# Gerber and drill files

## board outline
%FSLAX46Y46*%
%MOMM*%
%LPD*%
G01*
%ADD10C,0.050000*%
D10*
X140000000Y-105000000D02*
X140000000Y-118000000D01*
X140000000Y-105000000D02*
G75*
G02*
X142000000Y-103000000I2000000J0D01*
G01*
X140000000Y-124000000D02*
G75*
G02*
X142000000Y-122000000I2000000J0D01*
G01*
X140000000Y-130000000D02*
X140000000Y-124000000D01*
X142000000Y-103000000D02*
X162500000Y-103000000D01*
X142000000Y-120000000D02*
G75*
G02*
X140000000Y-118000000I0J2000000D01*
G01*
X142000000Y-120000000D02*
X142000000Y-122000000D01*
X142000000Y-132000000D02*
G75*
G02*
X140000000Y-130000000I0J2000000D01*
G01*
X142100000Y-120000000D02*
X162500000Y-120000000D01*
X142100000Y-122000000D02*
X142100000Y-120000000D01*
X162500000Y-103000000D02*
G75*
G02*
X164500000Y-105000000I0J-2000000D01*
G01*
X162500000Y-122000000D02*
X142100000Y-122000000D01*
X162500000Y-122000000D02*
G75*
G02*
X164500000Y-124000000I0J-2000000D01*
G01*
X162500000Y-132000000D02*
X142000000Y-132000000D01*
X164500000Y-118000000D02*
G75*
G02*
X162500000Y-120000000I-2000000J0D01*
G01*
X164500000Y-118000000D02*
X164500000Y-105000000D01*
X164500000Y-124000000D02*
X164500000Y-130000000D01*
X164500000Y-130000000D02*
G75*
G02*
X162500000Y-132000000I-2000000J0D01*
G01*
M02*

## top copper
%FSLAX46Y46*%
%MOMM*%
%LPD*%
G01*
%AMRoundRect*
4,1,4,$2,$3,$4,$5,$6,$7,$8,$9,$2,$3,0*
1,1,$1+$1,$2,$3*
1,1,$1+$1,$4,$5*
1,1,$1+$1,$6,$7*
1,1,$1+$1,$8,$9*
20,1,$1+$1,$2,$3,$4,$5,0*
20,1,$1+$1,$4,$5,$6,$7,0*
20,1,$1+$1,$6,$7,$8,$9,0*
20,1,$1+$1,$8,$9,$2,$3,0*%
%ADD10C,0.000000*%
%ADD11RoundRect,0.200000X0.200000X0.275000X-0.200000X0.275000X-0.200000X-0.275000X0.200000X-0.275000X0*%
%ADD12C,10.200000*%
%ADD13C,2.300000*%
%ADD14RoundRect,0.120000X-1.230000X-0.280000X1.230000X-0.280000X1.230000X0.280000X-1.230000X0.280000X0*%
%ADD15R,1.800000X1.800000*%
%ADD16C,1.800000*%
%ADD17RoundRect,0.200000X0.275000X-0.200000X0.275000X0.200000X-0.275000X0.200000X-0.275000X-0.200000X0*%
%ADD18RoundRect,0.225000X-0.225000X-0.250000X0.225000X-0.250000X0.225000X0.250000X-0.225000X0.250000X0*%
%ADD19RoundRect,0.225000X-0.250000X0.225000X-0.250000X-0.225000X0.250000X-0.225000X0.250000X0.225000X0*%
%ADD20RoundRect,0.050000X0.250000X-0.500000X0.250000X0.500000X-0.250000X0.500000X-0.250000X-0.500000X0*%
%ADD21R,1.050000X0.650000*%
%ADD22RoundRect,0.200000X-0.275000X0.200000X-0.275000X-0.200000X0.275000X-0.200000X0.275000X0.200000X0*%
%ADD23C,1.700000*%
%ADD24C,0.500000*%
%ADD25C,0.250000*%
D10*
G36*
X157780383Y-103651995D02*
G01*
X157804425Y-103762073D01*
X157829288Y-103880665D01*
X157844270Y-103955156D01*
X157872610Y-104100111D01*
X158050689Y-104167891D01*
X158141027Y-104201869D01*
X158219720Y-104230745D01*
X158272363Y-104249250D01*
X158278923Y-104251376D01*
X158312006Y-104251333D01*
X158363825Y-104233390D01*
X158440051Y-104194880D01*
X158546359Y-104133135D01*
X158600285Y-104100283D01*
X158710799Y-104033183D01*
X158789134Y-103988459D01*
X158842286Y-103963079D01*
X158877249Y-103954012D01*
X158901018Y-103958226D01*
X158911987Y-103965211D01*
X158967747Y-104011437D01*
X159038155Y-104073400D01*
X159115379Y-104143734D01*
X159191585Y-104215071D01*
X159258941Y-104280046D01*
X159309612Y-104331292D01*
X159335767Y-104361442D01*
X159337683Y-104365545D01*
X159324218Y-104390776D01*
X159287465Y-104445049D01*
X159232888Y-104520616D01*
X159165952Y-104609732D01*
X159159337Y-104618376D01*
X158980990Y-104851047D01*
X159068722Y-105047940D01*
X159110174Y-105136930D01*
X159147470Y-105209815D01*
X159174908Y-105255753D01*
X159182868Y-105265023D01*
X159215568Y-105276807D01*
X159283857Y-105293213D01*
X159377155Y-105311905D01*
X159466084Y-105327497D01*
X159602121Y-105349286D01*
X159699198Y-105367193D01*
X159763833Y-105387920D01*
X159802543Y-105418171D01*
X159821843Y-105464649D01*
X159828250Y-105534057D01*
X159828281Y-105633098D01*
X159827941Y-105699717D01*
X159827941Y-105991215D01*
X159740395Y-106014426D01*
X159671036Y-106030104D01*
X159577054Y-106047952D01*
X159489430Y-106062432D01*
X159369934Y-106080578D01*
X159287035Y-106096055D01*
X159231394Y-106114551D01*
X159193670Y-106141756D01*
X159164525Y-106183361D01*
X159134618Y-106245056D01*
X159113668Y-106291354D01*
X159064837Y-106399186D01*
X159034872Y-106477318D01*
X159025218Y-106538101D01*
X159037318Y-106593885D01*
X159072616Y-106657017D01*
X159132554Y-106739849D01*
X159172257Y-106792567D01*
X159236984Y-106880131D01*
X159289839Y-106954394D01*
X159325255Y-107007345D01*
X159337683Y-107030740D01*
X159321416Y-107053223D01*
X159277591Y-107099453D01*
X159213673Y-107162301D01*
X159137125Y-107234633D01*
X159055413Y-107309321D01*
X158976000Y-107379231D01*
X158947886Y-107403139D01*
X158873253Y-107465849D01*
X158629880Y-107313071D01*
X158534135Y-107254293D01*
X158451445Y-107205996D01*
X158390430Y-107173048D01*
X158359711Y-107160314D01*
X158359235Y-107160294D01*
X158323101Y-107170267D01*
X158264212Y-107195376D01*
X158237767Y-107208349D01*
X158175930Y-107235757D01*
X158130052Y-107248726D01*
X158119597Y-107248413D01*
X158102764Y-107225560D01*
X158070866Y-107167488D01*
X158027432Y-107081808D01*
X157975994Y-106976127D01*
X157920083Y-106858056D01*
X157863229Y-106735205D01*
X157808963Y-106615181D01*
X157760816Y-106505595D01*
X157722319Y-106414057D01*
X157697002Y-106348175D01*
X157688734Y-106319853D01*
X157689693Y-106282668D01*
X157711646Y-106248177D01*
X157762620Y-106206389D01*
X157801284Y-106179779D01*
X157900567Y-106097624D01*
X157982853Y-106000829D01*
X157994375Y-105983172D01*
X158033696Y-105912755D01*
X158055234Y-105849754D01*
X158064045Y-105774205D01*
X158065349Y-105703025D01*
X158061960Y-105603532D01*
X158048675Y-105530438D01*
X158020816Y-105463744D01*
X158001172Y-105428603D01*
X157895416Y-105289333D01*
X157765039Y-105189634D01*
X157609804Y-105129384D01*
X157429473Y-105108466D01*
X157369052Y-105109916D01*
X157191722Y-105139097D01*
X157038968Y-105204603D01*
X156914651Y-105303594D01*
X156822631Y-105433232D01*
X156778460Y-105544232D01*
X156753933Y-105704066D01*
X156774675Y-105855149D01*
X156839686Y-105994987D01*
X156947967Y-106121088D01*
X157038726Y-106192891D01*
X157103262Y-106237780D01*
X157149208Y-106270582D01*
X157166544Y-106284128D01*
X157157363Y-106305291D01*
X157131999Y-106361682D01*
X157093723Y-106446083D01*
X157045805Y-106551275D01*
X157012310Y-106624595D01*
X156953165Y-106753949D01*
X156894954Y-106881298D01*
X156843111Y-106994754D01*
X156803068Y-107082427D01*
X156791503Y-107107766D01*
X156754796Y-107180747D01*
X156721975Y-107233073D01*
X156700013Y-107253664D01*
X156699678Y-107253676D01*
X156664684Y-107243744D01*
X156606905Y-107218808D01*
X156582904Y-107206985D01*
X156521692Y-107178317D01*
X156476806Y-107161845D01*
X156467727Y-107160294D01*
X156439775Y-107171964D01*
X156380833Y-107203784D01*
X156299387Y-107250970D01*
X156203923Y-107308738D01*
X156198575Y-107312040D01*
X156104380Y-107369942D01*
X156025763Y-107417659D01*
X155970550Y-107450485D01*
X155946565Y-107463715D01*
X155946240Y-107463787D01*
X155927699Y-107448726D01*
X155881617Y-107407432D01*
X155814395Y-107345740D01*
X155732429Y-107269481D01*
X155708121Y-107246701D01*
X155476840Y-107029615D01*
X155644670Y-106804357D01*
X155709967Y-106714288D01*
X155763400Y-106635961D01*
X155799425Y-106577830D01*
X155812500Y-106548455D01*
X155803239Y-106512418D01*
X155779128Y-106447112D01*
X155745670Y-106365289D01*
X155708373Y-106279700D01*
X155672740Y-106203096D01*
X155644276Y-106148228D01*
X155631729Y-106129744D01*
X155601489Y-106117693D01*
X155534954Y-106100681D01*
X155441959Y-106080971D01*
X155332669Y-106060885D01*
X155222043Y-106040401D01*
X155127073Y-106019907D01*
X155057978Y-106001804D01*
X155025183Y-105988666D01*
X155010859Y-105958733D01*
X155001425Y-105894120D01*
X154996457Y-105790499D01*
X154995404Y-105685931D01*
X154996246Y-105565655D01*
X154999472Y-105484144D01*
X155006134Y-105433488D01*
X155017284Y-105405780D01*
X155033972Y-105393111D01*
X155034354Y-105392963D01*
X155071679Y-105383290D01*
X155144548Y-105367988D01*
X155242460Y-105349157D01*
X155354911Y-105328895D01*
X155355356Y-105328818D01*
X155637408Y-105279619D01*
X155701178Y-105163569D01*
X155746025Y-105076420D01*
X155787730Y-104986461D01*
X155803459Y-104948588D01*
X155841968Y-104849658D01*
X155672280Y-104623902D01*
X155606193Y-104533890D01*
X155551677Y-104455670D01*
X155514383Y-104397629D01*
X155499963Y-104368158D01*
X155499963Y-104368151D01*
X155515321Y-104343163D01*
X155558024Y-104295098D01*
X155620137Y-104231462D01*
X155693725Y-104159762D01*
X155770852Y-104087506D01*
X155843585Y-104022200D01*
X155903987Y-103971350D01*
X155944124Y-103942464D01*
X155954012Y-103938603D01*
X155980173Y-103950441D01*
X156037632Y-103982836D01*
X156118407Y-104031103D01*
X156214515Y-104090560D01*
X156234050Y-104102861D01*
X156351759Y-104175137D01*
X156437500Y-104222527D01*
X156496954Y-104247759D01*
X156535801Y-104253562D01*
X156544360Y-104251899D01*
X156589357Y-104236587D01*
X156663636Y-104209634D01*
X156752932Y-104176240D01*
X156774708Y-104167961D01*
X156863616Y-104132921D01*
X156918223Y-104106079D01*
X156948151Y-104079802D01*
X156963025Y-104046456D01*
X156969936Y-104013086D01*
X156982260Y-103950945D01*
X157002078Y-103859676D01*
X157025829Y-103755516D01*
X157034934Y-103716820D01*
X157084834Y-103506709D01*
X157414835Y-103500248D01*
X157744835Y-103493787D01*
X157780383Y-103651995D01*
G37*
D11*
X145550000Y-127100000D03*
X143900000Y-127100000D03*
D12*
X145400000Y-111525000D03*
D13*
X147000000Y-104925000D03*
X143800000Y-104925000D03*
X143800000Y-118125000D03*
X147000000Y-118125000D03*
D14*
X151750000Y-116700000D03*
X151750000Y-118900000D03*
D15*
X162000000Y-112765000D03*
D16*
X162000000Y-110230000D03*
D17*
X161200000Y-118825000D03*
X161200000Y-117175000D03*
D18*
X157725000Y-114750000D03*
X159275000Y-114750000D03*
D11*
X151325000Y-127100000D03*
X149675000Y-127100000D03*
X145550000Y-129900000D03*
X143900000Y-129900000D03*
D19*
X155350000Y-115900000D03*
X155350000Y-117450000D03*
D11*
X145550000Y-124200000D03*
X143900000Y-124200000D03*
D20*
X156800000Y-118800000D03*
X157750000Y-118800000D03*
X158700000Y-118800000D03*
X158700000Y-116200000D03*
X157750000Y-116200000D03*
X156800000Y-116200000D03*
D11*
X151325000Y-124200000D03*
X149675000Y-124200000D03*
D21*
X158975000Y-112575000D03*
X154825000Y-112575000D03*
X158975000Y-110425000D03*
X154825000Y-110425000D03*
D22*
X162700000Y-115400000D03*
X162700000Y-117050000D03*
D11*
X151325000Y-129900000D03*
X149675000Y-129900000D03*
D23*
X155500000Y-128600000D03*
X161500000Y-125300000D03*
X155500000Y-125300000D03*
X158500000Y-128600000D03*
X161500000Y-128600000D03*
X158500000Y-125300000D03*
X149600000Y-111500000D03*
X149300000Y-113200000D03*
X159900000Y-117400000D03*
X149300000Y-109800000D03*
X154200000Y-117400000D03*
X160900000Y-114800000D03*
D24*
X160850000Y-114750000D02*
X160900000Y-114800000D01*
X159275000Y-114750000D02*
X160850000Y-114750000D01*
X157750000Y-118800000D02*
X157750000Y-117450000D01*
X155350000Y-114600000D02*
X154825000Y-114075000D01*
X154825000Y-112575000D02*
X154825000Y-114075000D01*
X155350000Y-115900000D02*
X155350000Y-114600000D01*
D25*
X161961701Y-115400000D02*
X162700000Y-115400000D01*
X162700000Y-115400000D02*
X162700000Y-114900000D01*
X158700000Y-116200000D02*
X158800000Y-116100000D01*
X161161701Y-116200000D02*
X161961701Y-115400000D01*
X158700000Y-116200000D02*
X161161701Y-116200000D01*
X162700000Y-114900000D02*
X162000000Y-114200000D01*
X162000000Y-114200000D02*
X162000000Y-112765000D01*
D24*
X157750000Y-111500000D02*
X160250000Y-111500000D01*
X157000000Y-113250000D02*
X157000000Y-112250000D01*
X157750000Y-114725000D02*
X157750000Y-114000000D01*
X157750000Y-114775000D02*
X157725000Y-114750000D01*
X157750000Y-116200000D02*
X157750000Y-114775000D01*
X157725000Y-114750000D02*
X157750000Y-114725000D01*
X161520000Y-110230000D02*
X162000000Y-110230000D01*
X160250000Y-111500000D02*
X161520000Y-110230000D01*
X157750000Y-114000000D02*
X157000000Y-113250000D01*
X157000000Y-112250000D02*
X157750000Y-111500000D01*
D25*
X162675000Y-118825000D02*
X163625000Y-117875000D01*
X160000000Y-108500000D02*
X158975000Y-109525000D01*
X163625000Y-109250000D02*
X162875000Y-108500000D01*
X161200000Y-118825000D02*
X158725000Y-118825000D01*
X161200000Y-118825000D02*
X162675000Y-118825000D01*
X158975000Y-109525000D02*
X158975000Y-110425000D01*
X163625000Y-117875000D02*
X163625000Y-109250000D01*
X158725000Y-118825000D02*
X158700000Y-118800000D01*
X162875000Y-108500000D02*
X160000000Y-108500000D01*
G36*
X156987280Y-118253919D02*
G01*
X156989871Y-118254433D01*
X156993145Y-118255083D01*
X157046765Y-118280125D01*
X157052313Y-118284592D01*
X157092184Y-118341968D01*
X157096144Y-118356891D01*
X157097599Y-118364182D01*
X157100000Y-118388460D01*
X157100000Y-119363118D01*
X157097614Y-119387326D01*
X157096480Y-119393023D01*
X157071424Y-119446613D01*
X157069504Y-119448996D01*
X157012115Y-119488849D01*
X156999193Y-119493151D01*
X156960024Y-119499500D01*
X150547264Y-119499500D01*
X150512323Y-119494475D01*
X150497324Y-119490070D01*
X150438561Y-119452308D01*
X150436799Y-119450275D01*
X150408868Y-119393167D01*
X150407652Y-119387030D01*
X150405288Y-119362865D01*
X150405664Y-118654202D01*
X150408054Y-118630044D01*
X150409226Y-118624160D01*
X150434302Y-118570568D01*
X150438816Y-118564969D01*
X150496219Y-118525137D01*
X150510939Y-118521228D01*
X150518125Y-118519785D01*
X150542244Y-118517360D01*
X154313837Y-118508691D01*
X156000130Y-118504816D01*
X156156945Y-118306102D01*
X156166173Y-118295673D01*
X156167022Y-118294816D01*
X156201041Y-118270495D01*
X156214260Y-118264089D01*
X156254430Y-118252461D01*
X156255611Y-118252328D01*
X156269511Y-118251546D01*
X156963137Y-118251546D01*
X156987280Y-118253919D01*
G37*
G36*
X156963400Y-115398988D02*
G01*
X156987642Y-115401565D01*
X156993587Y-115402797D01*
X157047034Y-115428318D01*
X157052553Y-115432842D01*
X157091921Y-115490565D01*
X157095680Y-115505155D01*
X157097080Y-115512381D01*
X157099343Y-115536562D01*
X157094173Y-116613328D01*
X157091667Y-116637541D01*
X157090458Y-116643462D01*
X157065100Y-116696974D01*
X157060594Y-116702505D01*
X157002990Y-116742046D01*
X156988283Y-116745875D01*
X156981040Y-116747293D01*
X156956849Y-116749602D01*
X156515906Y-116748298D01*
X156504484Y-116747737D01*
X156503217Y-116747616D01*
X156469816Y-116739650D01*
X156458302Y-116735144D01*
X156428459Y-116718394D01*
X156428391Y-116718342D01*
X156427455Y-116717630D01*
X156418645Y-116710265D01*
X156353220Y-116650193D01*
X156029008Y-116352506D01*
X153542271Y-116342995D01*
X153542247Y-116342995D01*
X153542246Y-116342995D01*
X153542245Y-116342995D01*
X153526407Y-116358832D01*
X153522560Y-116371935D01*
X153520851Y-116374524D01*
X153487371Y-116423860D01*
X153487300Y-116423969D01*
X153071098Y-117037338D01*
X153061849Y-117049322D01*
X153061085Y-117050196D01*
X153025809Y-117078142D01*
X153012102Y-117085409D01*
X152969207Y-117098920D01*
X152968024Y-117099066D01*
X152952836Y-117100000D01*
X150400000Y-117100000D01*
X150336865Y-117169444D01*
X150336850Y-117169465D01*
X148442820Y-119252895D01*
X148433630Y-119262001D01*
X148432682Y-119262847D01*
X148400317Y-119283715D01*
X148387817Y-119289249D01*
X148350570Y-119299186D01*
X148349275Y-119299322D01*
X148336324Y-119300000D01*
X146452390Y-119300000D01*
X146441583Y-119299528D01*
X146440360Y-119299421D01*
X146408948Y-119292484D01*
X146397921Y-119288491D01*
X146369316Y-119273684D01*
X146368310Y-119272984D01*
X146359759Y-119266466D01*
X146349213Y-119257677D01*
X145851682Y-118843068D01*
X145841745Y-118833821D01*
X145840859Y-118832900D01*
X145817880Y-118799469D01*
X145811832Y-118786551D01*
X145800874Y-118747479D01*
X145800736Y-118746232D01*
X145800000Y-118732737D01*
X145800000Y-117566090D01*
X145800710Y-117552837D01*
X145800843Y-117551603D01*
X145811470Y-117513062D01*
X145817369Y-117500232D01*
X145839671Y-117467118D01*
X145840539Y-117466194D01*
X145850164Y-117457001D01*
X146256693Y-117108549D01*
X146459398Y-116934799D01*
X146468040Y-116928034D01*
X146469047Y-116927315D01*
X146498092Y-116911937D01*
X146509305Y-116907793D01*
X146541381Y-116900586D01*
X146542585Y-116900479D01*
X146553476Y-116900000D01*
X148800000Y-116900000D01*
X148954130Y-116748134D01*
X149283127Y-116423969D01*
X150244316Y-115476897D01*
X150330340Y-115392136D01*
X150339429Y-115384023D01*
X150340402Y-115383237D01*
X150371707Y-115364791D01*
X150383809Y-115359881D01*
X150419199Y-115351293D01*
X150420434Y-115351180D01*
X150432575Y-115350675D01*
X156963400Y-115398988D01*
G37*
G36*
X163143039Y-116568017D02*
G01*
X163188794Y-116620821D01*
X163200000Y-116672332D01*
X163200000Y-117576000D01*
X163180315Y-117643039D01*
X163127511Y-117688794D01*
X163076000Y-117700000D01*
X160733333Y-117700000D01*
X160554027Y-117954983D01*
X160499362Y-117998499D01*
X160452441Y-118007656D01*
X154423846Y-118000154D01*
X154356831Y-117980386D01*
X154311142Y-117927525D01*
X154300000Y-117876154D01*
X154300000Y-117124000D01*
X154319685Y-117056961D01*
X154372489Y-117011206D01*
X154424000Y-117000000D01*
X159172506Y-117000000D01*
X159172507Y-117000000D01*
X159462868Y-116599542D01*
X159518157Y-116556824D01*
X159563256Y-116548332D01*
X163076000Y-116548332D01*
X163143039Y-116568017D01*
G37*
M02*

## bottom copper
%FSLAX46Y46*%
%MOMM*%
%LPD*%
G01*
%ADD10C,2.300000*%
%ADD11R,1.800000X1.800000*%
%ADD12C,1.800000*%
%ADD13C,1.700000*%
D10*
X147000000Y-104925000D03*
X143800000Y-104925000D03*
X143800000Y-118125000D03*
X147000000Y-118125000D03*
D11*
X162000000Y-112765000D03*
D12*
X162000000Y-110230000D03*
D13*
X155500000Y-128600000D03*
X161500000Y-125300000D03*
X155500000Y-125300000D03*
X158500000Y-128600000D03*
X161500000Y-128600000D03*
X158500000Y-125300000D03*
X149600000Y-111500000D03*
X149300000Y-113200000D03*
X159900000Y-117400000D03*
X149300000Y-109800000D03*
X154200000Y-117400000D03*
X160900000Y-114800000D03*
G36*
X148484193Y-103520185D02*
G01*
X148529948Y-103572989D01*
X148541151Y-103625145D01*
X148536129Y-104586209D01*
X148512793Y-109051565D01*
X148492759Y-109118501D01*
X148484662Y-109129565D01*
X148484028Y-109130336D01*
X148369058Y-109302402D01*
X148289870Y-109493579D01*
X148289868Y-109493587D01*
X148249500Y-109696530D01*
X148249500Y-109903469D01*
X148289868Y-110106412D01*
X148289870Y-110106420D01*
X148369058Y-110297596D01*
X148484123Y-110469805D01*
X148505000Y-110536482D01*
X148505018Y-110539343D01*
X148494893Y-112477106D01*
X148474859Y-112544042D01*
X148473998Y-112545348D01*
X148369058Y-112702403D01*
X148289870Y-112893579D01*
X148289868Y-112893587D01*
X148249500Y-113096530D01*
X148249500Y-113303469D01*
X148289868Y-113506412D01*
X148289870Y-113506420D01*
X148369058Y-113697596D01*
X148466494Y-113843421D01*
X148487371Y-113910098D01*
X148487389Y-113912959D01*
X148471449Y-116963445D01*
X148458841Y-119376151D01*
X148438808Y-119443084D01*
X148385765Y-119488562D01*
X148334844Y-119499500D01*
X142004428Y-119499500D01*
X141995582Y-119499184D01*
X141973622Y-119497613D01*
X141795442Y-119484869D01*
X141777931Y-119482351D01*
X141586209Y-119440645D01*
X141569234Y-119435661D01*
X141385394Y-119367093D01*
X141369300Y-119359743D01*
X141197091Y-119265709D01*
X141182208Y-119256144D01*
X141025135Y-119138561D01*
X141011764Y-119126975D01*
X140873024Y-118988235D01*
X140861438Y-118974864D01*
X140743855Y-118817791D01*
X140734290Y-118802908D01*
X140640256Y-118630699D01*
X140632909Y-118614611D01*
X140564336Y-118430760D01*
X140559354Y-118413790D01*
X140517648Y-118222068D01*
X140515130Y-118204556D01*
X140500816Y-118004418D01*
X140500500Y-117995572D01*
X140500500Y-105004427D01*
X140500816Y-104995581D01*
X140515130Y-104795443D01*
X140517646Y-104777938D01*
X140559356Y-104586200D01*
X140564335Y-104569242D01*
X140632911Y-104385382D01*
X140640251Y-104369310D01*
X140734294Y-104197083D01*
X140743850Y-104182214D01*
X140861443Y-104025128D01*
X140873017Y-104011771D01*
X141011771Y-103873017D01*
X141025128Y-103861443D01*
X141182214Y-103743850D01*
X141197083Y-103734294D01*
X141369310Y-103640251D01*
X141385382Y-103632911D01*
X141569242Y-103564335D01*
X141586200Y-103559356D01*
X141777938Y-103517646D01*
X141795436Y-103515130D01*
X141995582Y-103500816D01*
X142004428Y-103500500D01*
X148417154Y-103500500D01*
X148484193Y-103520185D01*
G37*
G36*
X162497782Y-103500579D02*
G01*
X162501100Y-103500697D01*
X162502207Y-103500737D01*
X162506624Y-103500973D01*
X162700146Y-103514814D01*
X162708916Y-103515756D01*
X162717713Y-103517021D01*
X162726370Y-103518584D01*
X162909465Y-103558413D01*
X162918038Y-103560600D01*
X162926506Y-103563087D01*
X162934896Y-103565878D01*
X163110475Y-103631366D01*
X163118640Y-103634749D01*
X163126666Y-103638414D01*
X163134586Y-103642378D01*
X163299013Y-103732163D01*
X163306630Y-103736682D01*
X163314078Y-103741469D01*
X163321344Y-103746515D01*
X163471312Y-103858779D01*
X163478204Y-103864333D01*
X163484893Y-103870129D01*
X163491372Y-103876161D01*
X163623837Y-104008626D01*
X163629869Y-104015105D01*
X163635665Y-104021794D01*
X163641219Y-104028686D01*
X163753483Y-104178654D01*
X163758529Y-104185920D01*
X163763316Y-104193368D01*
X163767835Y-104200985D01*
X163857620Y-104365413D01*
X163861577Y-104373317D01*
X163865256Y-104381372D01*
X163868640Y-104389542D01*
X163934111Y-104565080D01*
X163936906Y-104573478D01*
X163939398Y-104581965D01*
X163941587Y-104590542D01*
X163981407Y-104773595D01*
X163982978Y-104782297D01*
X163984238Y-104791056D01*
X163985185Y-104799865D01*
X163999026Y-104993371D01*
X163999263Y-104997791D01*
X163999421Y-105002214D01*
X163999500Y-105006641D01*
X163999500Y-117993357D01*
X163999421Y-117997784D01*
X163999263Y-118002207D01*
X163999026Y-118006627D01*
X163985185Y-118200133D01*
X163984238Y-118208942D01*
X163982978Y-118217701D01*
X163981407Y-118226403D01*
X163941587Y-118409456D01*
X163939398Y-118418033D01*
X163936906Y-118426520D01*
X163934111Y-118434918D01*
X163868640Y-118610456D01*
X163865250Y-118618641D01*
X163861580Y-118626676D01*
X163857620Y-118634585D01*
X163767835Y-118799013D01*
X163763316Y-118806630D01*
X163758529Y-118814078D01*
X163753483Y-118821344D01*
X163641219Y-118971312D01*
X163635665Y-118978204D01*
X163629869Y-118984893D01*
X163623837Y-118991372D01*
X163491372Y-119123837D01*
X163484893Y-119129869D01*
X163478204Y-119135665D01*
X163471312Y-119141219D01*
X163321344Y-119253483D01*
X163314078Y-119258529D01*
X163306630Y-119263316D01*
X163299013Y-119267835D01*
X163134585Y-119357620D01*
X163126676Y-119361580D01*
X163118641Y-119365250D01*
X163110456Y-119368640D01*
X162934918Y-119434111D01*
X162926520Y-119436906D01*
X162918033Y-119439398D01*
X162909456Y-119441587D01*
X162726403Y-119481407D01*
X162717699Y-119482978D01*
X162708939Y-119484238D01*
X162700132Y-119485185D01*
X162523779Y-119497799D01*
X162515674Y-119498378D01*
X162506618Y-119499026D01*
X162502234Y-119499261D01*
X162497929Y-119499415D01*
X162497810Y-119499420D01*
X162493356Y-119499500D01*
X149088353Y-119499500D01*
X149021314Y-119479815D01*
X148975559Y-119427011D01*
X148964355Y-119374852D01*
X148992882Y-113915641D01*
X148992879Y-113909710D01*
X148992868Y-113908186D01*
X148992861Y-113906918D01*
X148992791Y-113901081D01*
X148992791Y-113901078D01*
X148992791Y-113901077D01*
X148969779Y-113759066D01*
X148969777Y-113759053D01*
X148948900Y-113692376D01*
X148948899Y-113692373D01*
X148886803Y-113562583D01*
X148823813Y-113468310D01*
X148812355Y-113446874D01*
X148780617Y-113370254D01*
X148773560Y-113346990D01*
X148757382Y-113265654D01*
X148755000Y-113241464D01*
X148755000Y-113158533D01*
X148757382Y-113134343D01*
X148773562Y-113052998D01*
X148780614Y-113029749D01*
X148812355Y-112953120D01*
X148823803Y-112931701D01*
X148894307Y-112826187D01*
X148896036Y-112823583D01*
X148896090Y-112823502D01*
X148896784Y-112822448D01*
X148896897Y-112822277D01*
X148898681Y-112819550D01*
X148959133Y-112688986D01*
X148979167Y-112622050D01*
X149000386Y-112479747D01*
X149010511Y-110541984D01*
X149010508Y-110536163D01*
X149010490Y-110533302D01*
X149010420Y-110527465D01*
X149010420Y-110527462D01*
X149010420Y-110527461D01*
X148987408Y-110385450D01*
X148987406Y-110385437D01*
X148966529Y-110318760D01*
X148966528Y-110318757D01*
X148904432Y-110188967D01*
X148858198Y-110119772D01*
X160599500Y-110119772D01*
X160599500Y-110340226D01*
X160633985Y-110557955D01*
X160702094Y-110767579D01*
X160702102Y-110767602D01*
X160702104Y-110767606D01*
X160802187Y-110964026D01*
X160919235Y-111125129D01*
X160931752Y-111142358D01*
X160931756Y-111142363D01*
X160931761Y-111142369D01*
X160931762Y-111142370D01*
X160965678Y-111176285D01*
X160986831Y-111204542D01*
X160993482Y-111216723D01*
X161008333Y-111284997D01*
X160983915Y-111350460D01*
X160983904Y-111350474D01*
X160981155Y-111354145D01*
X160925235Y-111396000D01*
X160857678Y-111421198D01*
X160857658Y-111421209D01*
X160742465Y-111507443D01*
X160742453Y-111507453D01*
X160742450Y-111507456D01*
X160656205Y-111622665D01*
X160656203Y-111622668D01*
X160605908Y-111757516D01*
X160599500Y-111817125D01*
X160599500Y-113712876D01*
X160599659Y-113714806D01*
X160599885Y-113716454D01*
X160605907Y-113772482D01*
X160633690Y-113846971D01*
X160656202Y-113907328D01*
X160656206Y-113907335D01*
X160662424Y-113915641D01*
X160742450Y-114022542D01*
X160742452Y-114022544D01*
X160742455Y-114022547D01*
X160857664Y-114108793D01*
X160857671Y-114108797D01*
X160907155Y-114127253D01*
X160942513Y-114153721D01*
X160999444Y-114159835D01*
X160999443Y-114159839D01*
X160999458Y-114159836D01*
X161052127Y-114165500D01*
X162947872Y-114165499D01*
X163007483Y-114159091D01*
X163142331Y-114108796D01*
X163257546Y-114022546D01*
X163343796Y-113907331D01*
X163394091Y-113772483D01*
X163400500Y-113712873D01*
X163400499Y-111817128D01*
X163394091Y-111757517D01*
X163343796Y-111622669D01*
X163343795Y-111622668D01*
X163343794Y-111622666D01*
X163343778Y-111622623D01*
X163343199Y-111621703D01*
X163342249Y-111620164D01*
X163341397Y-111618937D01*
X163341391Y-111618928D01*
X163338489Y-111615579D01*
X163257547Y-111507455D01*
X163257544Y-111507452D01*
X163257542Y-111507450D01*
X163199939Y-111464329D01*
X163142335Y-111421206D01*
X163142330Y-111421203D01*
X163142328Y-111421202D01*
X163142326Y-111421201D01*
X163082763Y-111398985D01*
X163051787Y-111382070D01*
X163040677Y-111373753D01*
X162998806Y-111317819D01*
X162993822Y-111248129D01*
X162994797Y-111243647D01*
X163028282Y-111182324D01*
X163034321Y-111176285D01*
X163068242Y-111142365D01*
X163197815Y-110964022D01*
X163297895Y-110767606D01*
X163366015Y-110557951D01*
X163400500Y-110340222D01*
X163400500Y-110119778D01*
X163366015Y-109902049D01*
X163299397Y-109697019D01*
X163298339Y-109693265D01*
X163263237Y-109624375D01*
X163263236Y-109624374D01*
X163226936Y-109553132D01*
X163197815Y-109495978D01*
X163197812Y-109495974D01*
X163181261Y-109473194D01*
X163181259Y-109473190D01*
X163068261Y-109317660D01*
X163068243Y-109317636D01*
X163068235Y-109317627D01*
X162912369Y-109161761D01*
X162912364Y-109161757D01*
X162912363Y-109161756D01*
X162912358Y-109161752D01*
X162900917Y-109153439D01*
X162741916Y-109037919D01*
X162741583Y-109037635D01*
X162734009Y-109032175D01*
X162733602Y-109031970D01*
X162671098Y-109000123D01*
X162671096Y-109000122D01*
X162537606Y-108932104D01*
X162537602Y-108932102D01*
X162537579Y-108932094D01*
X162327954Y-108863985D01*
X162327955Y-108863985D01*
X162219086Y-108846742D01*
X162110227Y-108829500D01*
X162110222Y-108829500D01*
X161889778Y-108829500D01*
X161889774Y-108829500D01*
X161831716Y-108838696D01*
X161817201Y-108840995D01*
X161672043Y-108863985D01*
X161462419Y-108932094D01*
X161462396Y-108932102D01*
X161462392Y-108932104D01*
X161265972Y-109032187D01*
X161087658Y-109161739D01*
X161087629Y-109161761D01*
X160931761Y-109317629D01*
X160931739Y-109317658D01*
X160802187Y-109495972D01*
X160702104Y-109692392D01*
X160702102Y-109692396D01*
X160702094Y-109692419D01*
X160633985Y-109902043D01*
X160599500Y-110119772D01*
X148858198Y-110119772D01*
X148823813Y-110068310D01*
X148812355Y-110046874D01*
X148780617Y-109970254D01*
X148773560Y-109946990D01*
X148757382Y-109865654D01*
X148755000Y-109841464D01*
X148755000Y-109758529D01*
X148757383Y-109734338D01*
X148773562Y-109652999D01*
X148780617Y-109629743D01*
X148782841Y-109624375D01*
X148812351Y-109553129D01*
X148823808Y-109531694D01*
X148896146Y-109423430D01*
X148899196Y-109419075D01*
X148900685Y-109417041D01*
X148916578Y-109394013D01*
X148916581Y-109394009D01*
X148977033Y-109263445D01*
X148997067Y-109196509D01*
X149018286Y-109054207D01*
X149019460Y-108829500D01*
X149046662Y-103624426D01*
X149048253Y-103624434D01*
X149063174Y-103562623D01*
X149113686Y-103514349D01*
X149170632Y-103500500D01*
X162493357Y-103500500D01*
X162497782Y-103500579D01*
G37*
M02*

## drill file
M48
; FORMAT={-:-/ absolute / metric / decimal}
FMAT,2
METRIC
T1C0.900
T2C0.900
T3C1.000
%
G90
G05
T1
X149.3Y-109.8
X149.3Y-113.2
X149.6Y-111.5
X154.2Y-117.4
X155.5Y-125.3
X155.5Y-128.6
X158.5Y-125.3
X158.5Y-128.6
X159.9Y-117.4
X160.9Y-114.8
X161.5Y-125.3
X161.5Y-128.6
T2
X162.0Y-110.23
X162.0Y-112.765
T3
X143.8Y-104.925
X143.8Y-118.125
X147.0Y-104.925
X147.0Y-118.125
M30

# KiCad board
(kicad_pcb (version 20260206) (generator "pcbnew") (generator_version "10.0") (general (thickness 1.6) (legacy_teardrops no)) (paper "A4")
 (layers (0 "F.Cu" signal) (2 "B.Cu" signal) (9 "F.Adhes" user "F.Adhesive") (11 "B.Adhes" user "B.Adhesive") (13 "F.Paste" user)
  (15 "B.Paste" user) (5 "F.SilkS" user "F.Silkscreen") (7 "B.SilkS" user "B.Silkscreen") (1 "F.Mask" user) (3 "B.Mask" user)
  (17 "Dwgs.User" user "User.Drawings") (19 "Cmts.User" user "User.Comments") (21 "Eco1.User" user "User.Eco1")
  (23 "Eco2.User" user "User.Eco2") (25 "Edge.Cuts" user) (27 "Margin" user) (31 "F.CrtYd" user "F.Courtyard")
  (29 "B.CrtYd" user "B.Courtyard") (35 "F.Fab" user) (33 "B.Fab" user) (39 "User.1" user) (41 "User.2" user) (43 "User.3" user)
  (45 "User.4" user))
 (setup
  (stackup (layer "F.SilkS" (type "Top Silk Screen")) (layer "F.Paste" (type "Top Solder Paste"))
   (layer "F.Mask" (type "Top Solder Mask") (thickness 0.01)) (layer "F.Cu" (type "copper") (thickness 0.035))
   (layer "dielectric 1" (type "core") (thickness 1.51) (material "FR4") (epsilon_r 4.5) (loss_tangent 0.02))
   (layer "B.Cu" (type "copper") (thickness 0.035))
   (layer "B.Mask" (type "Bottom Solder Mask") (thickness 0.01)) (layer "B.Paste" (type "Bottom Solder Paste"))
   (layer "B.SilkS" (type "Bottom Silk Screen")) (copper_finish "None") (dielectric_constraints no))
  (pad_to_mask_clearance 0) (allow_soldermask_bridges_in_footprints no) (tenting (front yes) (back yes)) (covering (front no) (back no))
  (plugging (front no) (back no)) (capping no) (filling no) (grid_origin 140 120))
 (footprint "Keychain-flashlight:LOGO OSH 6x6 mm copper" (layer "F.Cu") (at 157.4 106.6)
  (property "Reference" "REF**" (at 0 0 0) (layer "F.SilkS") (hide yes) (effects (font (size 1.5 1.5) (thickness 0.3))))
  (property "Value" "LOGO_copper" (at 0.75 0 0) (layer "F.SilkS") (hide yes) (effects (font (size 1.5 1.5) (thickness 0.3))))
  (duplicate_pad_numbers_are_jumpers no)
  (fp_poly
   (pts (xy 0.380383 -2.948005) (xy 0.404425 -2.837927) (xy 0.429288 -2.719335) (xy 0.44427 -2.644844) (xy 0.47261 -2.499889)
    (xy 0.650689 -2.432109) (xy 0.741027 -2.398131) (xy 0.81972 -2.369255) (xy 0.872363 -2.35075) (xy 0.878923 -2.348624)
    (xy 0.912006 -2.348667) (xy 0.963825 -2.36661) (xy 1.040051 -2.40512) (xy 1.146359 -2.466865) (xy 1.200285 -2.499717)
    (xy 1.310799 -2.566817) (xy 1.389134 -2.611541) (xy 1.442286 -2.636921) (xy 1.477249 -2.645988) (xy 1.501018 -2.641774)
    (xy 1.511987 -2.634789) (xy 1.567747 -2.588563) (xy 1.638155 -2.5266) (xy 1.715379 -2.456266) (xy 1.791585 -2.384929)
    (xy 1.858941 -2.319954) (xy 1.909612 -2.268708) (xy 1.935767 -2.238558) (xy 1.937683 -2.234455) (xy 1.924218 -2.209224)
    (xy 1.887465 -2.154951) (xy 1.832888 -2.079384) (xy 1.765952 -1.990268) (xy 1.759337 -1.981624) (xy 1.58099 -1.748953)
    (xy 1.668722 -1.55206) (xy 1.710174 -1.46307) (xy 1.74747 -1.390185) (xy 1.774908 -1.344247) (xy 1.782868 -1.334977)
    (xy 1.815568 -1.323193) (xy 1.883857 -1.306787) (xy 1.977155 -1.288095) (xy 2.066084 -1.272503) (xy 2.202121 -1.250714)
    (xy 2.299198 -1.232807) (xy 2.363833 -1.21208) (xy 2.402543 -1.181829) (xy 2.421843 -1.135351) (xy 2.42825 -1.065943)
    (xy 2.428281 -0.966902) (xy 2.427941 -0.900283) (xy 2.427941 -0.608785) (xy 2.340395 -0.585574) (xy 2.271036 -0.569896)
    (xy 2.177054 -0.552048) (xy 2.08943 -0.537568) (xy 1.969934 -0.519422) (xy 1.887035 -0.503945) (xy 1.831394 -0.485449)
    (xy 1.79367 -0.458244) (xy 1.764525 -0.416639) (xy 1.734618 -0.354944) (xy 1.713668 -0.308646) (xy 1.664837 -0.200814)
    (xy 1.634872 -0.122682) (xy 1.625218 -0.061899) (xy 1.637318 -0.006115) (xy 1.672616 0.057017) (xy 1.732554 0.139849)
    (xy 1.772257 0.192567) (xy 1.836984 0.280131) (xy 1.889839 0.354394) (xy 1.925255 0.407345) (xy 1.937683 0.43074) (xy 1.921416 0.453223)
    (xy 1.877591 0.499453) (xy 1.813673 0.562301) (xy 1.737125 0.634633) (xy 1.655413 0.709321) (xy 1.576 0.779231) (xy 1.547886 0.803139)
    (xy 1.473253 0.865849) (xy 1.22988 0.713071) (xy 1.134135 0.654293) (xy 1.051445 0.605996) (xy 0.99043 0.573048) (xy 0.959711 0.560314)
    (xy 0.959235 0.560294) (xy 0.923101 0.570267) (xy 0.864212 0.595376) (xy 0.837767 0.608349) (xy 0.77593 0.635757) (xy 0.730052 0.648726)
    (xy 0.719597 0.648413) (xy 0.702764 0.62556) (xy 0.670866 0.567488) (xy 0.627432 0.481808) (xy 0.575994 0.376127) (xy 0.520083 0.258056)
    (xy 0.463229 0.135205) (xy 0.408963 0.015181) (xy 0.360816 -0.094405) (xy 0.322319 -0.185943) (xy 0.297002 -0.251825)
    (xy 0.288734 -0.280147) (xy 0.289693 -0.317332) (xy 0.311646 -0.351823) (xy 0.36262 -0.393611) (xy 0.401284 -0.420221)
    (xy 0.500567 -0.502376) (xy 0.582853 -0.599171) (xy 0.594375 -0.616828) (xy 0.633696 -0.687245) (xy 0.655234 -0.750246)
    (xy 0.664045 -0.825795) (xy 0.665349 -0.896975) (xy 0.66196 -0.996468) (xy 0.648675 -1.069562) (xy 0.620816 -1.136256)
    (xy 0.601172 -1.171397) (xy 0.495416 -1.310667) (xy 0.365039 -1.410366) (xy 0.209804 -1.470616) (xy 0.029473 -1.491534)
    (xy -0.030948 -1.490084) (xy -0.208278 -1.460903) (xy -0.361032 -1.395397) (xy -0.485349 -1.296406) (xy -0.577369 -1.166768)
    (xy -0.62154 -1.055768) (xy -0.646067 -0.895934) (xy -0.625325 -0.744851) (xy -0.560314 -0.605013) (xy -0.452033 -0.478912)
    (xy -0.361274 -0.407109) (xy -0.296738 -0.36222) (xy -0.250792 -0.329418) (xy -0.233456 -0.315872) (xy -0.242637 -0.294709)
    (xy -0.268001 -0.238318) (xy -0.306277 -0.153917) (xy -0.354195 -0.048725) (xy -0.38769 0.024595) (xy -0.446835 0.153949)
    (xy -0.505046 0.281298) (xy -0.556889 0.394754) (xy -0.596932 0.482427) (xy -0.608497 0.507766) (xy -0.645204 0.580747)
    (xy -0.678025 0.633073) (xy -0.699987 0.653664) (xy -0.700322 0.653676) (xy -0.735316 0.643744) (xy -0.793095 0.618808)
    (xy -0.817096 0.606985) (xy -0.878308 0.578317) (xy -0.923194 0.561845) (xy -0.932273 0.560294) (xy -0.960225 0.571964)
    (xy -1.019167 0.603784) (xy -1.100613 0.65097) (xy -1.196077 0.708738) (xy -1.201425 0.71204) (xy -1.29562 0.769942)
    (xy -1.374237 0.817659) (xy -1.42945 0.850485) (xy -1.453435 0.863715) (xy -1.45376 0.863787) (xy -1.472301 0.848726)
    (xy -1.518383 0.807432) (xy -1.585605 0.74574) (xy -1.667571 0.669481) (xy -1.691879 0.646701) (xy -1.92316 0.429615)
    (xy -1.75533 0.204357) (xy -1.690033 0.114288) (xy -1.6366 0.035961) (xy -1.600575 -0.02217) (xy -1.5875 -0.051545)
    (xy -1.596761 -0.087582) (xy -1.620872 -0.152888) (xy -1.65433 -0.234711) (xy -1.691627 -0.3203) (xy -1.72726 -0.396904)
    (xy -1.755724 -0.451772) (xy -1.768271 -0.470256) (xy -1.798511 -0.482307) (xy -1.865046 -0.499319) (xy -1.958041 -0.519029)
    (xy -2.067331 -0.539115) (xy -2.177957 -0.559599) (xy -2.272927 -0.580093) (xy -2.342022 -0.598196) (xy -2.374817 -0.611334)
    (xy -2.389141 -0.641267) (xy -2.398575 -0.70588) (xy -2.403543 -0.809501) (xy -2.404596 -0.914069) (xy -2.403754 -1.034345)
    (xy -2.400528 -1.115856) (xy -2.393866 -1.166512) (xy -2.382716 -1.19422) (xy -2.366028 -1.206889) (xy -2.365646 -1.207037)
    (xy -2.328321 -1.21671) (xy -2.255452 -1.232012) (xy -2.15754 -1.250843) (xy -2.045089 -1.271105) (xy -2.044644 -1.271182)
    (xy -1.762592 -1.320381) (xy -1.698822 -1.436431) (xy -1.653975 -1.52358) (xy -1.61227 -1.613539) (xy -1.596541 -1.651412)
    (xy -1.558032 -1.750342) (xy -1.72772 -1.976098) (xy -1.793807 -2.06611) (xy -1.848323 -2.14433) (xy -1.885617 -2.202371)
    (xy -1.900037 -2.231842) (xy -1.900037 -2.231849) (xy -1.884679 -2.256837) (xy -1.841976 -2.304902) (xy -1.779863 -2.368538)
    (xy -1.706275 -2.440238) (xy -1.629148 -2.512494) (xy -1.556415 -2.5778) (xy -1.496013 -2.62865) (xy -1.455876 -2.657536)
    (xy -1.445988 -2.661397) (xy -1.419827 -2.649559) (xy -1.362368 -2.617164) (xy -1.281593 -2.568897) (xy -1.185485 -2.50944)
    (xy -1.16595 -2.497139) (xy -1.048241 -2.424863) (xy -0.9625 -2.377473) (xy -0.903046 -2.352241) (xy -0.864199 -2.346438)
    (xy -0.85564 -2.348101) (xy -0.810643 -2.363413) (xy -0.736364 -2.390366) (xy -0.647068 -2.42376) (xy -0.625292 -2.432039)
    (xy -0.536384 -2.467079) (xy -0.481777 -2.493921) (xy -0.451849 -2.520198) (xy -0.436975 -2.553544) (xy -0.430064 -2.586914)
    (xy -0.41774 -2.649055) (xy -0.397922 -2.740324) (xy -0.374171 -2.844484) (xy -0.365066 -2.88318) (xy -0.315166 -3.093291)
    (xy 0.014835 -3.099752) (xy 0.344835 -3.106213))
   (stroke (width 0) (type solid)) (fill yes) (layer "F.Cu")))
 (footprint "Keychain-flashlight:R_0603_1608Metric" (layer "F.Cu") (at 144.725 127.1 180)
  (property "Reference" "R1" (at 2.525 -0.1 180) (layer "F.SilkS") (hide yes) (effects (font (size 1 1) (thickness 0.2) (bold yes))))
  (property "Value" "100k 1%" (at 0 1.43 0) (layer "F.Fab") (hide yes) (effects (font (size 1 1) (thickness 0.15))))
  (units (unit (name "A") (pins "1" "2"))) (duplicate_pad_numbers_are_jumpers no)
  (pad "1" smd roundrect (at -0.825 0 180) (size 0.8 0.95) (layers "F.Cu" "F.Mask" "F.Paste") (roundrect_rratio 0.25) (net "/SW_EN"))
  (pad "2" smd roundrect (at 0.825 0 180) (size 0.8 0.95) (layers "F.Cu" "F.Mask" "F.Paste") (roundrect_rratio 0.25) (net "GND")))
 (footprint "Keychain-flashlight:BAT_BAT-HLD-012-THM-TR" (layer "F.Cu") (at 145.4 111.525 -90)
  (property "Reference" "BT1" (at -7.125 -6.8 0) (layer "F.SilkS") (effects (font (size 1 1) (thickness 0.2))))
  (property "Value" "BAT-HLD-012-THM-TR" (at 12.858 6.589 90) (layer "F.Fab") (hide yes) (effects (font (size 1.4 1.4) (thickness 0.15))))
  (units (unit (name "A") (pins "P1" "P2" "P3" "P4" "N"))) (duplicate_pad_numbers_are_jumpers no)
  (pad "N" smd circle (at 0 0 270) (size 10.2 10.2) (layers "F.Cu" "F.Mask") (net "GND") (solder_mask_margin 0.102))
  (pad "P1" thru_hole circle (at -6.6 -1.6 270) (size 2.3 2.3) (drill 1) (layers "*.Cu" "*.Mask") (remove_unused_layers no) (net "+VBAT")
   (solder_mask_margin 0.102))
  (pad "P2" thru_hole circle (at -6.6 1.6 270) (size 2.3 2.3) (drill 1) (layers "*.Cu" "*.Mask") (remove_unused_layers no) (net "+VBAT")
   (solder_mask_margin 0.102))
  (pad "P3" thru_hole circle (at 6.6 1.6 270) (size 2.3 2.3) (drill 1) (layers "*.Cu" "*.Mask") (remove_unused_layers no) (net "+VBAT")
   (solder_mask_margin 0.102))
  (pad "P4" thru_hole circle (at 6.6 -1.6 270) (size 2.3 2.3) (drill 1) (layers "*.Cu" "*.Mask") (remove_unused_layers no) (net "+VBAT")
   (solder_mask_margin 0.102)))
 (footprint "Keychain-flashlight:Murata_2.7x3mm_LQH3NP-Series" (layer "F.Cu") (at 151.75 117.8 -90)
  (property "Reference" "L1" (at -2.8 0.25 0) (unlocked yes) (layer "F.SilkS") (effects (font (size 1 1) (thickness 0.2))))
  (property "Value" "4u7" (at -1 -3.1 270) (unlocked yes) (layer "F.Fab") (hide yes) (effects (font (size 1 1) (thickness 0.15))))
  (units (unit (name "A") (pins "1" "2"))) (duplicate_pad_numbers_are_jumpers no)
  (pad "1" smd roundrect (at -1.1 0) (size 2.7 0.8) (layers "F.Cu" "F.Mask" "F.Paste") (roundrect_rratio 0.15) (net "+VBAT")
   (thermal_bridge_angle 45))
  (pad "2" smd roundrect (at 1.1 0) (size 2.7 0.8) (layers "F.Cu" "F.Mask" "F.Paste") (roundrect_rratio 0.15) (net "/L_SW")
   (thermal_bridge_angle 45)))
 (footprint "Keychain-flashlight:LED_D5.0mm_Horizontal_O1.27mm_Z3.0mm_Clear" (layer "F.Cu") (at 162 112.77 90)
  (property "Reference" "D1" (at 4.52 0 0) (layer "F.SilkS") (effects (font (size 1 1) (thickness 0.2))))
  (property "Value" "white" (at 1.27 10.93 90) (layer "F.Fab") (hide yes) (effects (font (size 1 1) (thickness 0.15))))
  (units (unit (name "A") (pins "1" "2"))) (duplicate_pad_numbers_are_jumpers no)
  (pad "1" thru_hole rect (at 0.005 0 90) (size 1.8 1.8) (drill 0.9) (layers "*.Cu" "*.Mask") (remove_unused_layers no) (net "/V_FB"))
  (pad "2" thru_hole circle (at 2.54 0 90) (size 1.8 1.8) (drill 0.9) (layers "*.Cu" "*.Mask") (remove_unused_layers no) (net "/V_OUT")))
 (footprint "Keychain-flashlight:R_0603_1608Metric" (layer "F.Cu") (at 161.2 118 90)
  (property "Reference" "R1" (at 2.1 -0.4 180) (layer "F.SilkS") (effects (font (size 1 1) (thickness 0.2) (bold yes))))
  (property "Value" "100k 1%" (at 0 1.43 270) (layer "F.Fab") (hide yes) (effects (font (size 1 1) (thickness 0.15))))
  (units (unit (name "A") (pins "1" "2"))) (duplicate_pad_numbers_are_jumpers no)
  (pad "1" smd roundrect (at -0.825 0 90) (size 0.8 0.95) (layers "F.Cu" "F.Mask" "F.Paste") (roundrect_rratio 0.25) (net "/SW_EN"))
  (pad "2" smd roundrect (at 0.825 0 90) (size 0.8 0.95) (layers "F.Cu" "F.Mask" "F.Paste") (roundrect_rratio 0.25) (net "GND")))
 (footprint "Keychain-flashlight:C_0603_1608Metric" (layer "F.Cu") (at 158.5 114.75)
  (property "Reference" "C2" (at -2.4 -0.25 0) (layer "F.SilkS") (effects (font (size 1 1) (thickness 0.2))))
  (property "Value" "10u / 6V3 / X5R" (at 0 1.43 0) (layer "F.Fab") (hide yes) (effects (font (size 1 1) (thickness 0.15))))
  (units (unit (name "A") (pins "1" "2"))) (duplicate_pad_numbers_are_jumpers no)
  (pad "1" smd roundrect (at -0.775 0) (size 0.9 0.95) (layers "F.Cu" "F.Mask" "F.Paste") (roundrect_rratio 0.25) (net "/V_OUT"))
  (pad "2" smd roundrect (at 0.775 0) (size 0.9 0.95) (layers "F.Cu" "F.Mask" "F.Paste") (roundrect_rratio 0.25) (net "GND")))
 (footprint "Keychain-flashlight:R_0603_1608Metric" (layer "F.Cu") (at 150.5 127.1 180)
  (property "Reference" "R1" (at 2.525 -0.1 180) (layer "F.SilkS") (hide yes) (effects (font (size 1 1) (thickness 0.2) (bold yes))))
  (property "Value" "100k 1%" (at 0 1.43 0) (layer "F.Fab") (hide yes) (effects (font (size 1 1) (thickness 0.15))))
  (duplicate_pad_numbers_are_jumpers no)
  (pad "1" smd roundrect (at -0.825 0 180) (size 0.8 0.95) (layers "F.Cu" "F.Mask" "F.Paste") (roundrect_rratio 0.25))
  (pad "2" smd roundrect (at 0.825 0 180) (size 0.8 0.95) (layers "F.Cu" "F.Mask" "F.Paste") (roundrect_rratio 0.25)))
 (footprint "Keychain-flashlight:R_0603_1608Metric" (layer "F.Cu") (at 144.725 129.9 180)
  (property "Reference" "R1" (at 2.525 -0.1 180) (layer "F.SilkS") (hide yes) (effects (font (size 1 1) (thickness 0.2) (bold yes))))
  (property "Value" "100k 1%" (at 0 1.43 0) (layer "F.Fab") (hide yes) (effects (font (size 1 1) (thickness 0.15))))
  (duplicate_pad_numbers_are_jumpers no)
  (pad "1" smd roundrect (at -0.825 0 180) (size 0.8 0.95) (layers "F.Cu" "F.Mask" "F.Paste") (roundrect_rratio 0.25))
  (pad "2" smd roundrect (at 0.825 0 180) (size 0.8 0.95) (layers "F.Cu" "F.Mask" "F.Paste") (roundrect_rratio 0.25)))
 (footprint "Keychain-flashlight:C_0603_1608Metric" (layer "F.Cu") (at 155.35 116.675 -90)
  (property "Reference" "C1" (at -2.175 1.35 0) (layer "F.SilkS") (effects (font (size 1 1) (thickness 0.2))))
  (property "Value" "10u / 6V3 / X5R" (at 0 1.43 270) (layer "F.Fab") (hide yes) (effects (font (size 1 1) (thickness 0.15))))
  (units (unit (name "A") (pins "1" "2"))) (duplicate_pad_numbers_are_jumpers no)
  (pad "1" smd roundrect (at -0.775 0 270) (size 0.9 0.95) (layers "F.Cu" "F.Mask" "F.Paste") (roundrect_rratio 0.25) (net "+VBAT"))
  (pad "2" smd roundrect (at 0.775 0 270) (size 0.9 0.95) (layers "F.Cu" "F.Mask" "F.Paste") (roundrect_rratio 0.25) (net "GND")))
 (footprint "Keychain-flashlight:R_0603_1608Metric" (layer "F.Cu") (at 144.725 124.2 180)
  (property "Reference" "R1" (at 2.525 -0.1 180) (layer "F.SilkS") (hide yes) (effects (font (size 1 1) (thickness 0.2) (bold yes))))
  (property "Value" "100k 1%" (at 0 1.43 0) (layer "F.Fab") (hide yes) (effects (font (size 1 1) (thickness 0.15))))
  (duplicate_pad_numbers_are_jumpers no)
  (pad "1" smd roundrect (at -0.825 0 180) (size 0.8 0.95) (layers "F.Cu" "F.Mask" "F.Paste") (roundrect_rratio 0.25))
  (pad "2" smd roundrect (at 0.825 0 180) (size 0.8 0.95) (layers "F.Cu" "F.Mask" "F.Paste") (roundrect_rratio 0.25)))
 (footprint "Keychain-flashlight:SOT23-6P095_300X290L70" (layer "F.Cu") (at 157.75 117.5 90)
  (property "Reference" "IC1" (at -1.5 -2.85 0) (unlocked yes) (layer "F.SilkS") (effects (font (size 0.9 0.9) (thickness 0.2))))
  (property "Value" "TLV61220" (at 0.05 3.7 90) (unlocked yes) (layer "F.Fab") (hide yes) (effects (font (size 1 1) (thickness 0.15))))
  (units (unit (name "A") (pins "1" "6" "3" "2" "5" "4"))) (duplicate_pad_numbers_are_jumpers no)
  (pad "1" smd roundrect (at -1.3 -0.95 90) (size 1.1 0.6) (layers "F.Cu" "F.Mask" "F.Paste") (roundrect_rratio 0.08333333333) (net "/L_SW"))
  (pad "2" smd roundrect (at -1.3 0 90) (size 1.1 0.6) (layers "F.Cu" "F.Mask" "F.Paste") (roundrect_rratio 0.08333333333) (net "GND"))
  (pad "3" smd roundrect (at -1.3 0.95 90) (size 1.1 0.6) (layers "F.Cu" "F.Mask" "F.Paste") (roundrect_rratio 0.08333333333) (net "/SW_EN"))
  (pad "4" smd roundrect (at 1.3 0.95 90) (size 1.1 0.6) (layers "F.Cu" "F.Mask" "F.Paste") (roundrect_rratio 0.08333333333) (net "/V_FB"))
  (pad "5" smd roundrect (at 1.3 0 90) (size 1.1 0.6) (layers "F.Cu" "F.Mask" "F.Paste") (roundrect_rratio 0.08333333333) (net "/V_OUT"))
  (pad "6" smd roundrect (at 1.3 -0.95 90) (size 1.1 0.6) (layers "F.Cu" "F.Mask" "F.Paste") (roundrect_rratio 0.08333333333) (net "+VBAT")))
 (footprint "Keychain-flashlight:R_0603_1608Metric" (layer "F.Cu") (at 150.5 124.2 180)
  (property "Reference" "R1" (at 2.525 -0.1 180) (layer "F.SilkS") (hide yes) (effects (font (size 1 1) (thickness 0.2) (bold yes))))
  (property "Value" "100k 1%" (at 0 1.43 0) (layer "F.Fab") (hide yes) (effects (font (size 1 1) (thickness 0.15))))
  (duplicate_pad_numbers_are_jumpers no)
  (pad "1" smd roundrect (at -0.825 0 180) (size 0.8 0.95) (layers "F.Cu" "F.Mask" "F.Paste") (roundrect_rratio 0.25))
  (pad "2" smd roundrect (at 0.825 0 180) (size 0.8 0.95) (layers "F.Cu" "F.Mask" "F.Paste") (roundrect_rratio 0.25)))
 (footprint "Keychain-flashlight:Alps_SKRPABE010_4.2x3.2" (layer "F.Cu") (at 156.9 111.5 180)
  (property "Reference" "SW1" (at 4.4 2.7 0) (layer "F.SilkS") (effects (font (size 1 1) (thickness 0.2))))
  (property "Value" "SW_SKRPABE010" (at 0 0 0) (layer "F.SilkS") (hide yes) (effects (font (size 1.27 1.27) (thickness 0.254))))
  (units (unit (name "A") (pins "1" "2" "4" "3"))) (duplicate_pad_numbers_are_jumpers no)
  (pad "1" smd rect (at -2.075 -1.075 270) (size 0.65 1.05) (layers "F.Cu" "F.Mask" "F.Paste") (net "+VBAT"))
  (pad "2" smd rect (at 2.075 -1.075 270) (size 0.65 1.05) (layers "F.Cu" "F.Mask" "F.Paste") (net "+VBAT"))
  (pad "3" smd rect (at -2.075 1.075 270) (size 0.65 1.05) (layers "F.Cu" "F.Mask" "F.Paste") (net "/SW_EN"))
  (pad "4" smd rect (at 2.075 1.075 270) (size 0.65 1.05) (layers "F.Cu" "F.Mask" "F.Paste") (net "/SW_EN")))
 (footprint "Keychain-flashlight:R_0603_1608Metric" (layer "F.Cu") (at 162.7 116.225 -90)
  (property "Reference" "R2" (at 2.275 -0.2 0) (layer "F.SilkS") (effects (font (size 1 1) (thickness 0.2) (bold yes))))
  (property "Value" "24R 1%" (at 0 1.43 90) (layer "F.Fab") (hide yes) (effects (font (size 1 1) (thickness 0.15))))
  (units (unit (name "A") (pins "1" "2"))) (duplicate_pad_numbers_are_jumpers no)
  (pad "1" smd roundrect (at -0.825 0 270) (size 0.8 0.95) (layers "F.Cu" "F.Mask" "F.Paste") (roundrect_rratio 0.25) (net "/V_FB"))
  (pad "2" smd roundrect (at 0.825 0 270) (size 0.8 0.95) (layers "F.Cu" "F.Mask" "F.Paste") (roundrect_rratio 0.25) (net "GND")))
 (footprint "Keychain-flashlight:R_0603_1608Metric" (layer "F.Cu") (at 150.5 129.9 180)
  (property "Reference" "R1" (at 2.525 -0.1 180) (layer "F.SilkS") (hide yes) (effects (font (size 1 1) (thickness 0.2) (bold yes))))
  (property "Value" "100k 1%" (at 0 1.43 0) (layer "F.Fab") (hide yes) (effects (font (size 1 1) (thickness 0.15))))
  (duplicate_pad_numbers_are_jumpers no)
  (pad "1" smd roundrect (at -0.825 0 180) (size 0.8 0.95) (layers "F.Cu" "F.Mask" "F.Paste") (roundrect_rratio 0.25))
  (pad "2" smd roundrect (at 0.825 0 180) (size 0.8 0.95) (layers "F.Cu" "F.Mask" "F.Paste") (roundrect_rratio 0.25)))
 (gr_line (start 140 105) (end 140 118) (stroke (width 0.05) (type default)) (layer "Edge.Cuts"))
 (gr_arc (start 140 105) (mid 140.585786 103.585786) (end 142 103) (stroke (width 0.05) (type default)) (layer "Edge.Cuts"))
 (gr_arc (start 140 124) (mid 140.585786 122.585786) (end 142 122) (stroke (width 0.05) (type default)) (layer "Edge.Cuts"))
 (gr_line (start 140 130) (end 140 124) (stroke (width 0.05) (type default)) (layer "Edge.Cuts"))
 (gr_line (start 142 103) (end 162.5 103) (stroke (width 0.05) (type default)) (layer "Edge.Cuts"))
 (gr_arc (start 142 120) (mid 140.585786 119.414214) (end 140 118) (stroke (width 0.05) (type default)) (layer "Edge.Cuts"))
 (gr_line (start 142 120) (end 142 122) (stroke (width 0.05) (type default)) (layer "Edge.Cuts"))
 (gr_arc (start 142 132) (mid 140.585786 131.414214) (end 140 130) (stroke (width 0.05) (type default)) (layer "Edge.Cuts"))
 (gr_line (start 142.1 120) (end 162.5 120) (stroke (width 0.05) (type default)) (layer "Edge.Cuts"))
 (gr_line (start 142.1 122) (end 142.1 120) (stroke (width 0.05) (type default)) (layer "Edge.Cuts"))
 (gr_arc (start 162.5 103) (mid 163.914214 103.585786) (end 164.5 105) (stroke (width 0.05) (type default)) (layer "Edge.Cuts"))
 (gr_line (start 162.5 122) (end 142.1 122) (stroke (width 0.05) (type default)) (layer "Edge.Cuts"))
 (gr_arc (start 162.5 122) (mid 163.914214 122.585786) (end 164.5 124) (stroke (width 0.05) (type default)) (layer "Edge.Cuts"))
 (gr_line (start 162.5 132) (end 142 132) (stroke (width 0.05) (type default)) (layer "Edge.Cuts"))
 (gr_arc (start 164.5 118) (mid 163.914214 119.414214) (end 162.5 120) (stroke (width 0.05) (type default)) (layer "Edge.Cuts"))
 (gr_line (start 164.5 118) (end 164.5 105) (stroke (width 0.05) (type default)) (layer "Edge.Cuts"))
 (gr_line (start 164.5 124) (end 164.5 130) (stroke (width 0.05) (type default)) (layer "Edge.Cuts"))
 (gr_arc (start 164.5 130) (mid 163.914214 131.414214) (end 162.5 132) (stroke (width 0.05) (type default)) (layer "Edge.Cuts"))
 (via (at 155.5 128.6) (size 1.7) (drill 0.9) (layers "F.Cu" "B.Cu") (free yes) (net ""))
 (via (at 161.5 125.3) (size 1.7) (drill 0.9) (layers "F.Cu" "B.Cu") (free yes) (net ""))
 (via (at 155.5 125.3) (size 1.7) (drill 0.9) (layers "F.Cu" "B.Cu") (free yes) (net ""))
 (via (at 158.5 128.6) (size 1.7) (drill 0.9) (layers "F.Cu" "B.Cu") (free yes) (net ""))
 (via (at 161.5 128.6) (size 1.7) (drill 0.9) (layers "F.Cu" "B.Cu") (free yes) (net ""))
 (via (at 158.5 125.3) (size 1.7) (drill 0.9) (layers "F.Cu" "B.Cu") (free yes) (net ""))
 (segment (start 160.85 114.75) (end 160.9 114.8) (width 0.5) (layer "F.Cu") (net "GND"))
 (segment (start 159.275 114.75) (end 160.85 114.75) (width 0.5) (layer "F.Cu") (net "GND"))
 (segment (start 157.75 118.8) (end 157.75 117.45) (width 0.5) (layer "F.Cu") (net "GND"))
 (via (at 149.6 111.5) (size 1.7) (drill 0.9) (layers "F.Cu" "B.Cu") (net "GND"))
 (via (at 149.3 113.2) (size 1.7) (drill 0.9) (layers "F.Cu" "B.Cu") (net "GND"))
 (via (at 159.9 117.4) (size 1.7) (drill 0.9) (layers "F.Cu" "B.Cu") (free yes) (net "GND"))
 (via (at 149.3 109.8) (size 1.7) (drill 0.9) (layers "F.Cu" "B.Cu") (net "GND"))
 (via (at 154.2 117.4) (size 1.7) (drill 0.9) (layers "F.Cu" "B.Cu") (free yes) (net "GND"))
 (via (at 160.9 114.8) (size 1.7) (drill 0.9) (layers "F.Cu" "B.Cu") (free yes) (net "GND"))
 (segment (start 155.35 114.6) (end 154.825 114.075) (width 0.5) (layer "F.Cu") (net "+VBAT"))
 (segment (start 154.825 112.575) (end 154.825 114.075) (width 0.5) (layer "F.Cu") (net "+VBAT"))
 (segment (start 155.35 115.9) (end 155.35 114.6) (width 0.5) (layer "F.Cu") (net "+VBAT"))
 (segment (start 161.961701 115.4) (end 162.7 115.4) (width 0.25) (layer "F.Cu") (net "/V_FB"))
 (segment (start 162.7 115.4) (end 162.7 114.9) (width 0.25) (layer "F.Cu") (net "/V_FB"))
 (segment (start 158.7 116.2) (end 158.8 116.1) (width 0.25) (layer "F.Cu") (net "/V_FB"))
 (segment (start 161.161701 116.2) (end 161.961701 115.4) (width 0.25) (layer "F.Cu") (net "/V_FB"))
 (segment (start 158.7 116.2) (end 161.161701 116.2) (width 0.25) (layer "F.Cu") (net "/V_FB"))
 (segment (start 162.7 114.9) (end 162 114.2) (width 0.25) (layer "F.Cu") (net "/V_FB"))
 (segment (start 162 114.2) (end 162 112.765) (width 0.25) (layer "F.Cu") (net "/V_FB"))
 (segment (start 157.75 111.5) (end 160.25 111.5) (width 0.5) (layer "F.Cu") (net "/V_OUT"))
 (segment (start 157 113.25) (end 157 112.25) (width 0.5) (layer "F.Cu") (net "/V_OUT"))
 (segment (start 157.75 114.725) (end 157.75 114) (width 0.5) (layer "F.Cu") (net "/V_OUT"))
 (segment (start 157.75 114.775) (end 157.725 114.75) (width 0.5) (layer "F.Cu") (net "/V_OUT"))
 (segment (start 157.75 116.2) (end 157.75 114.775) (width 0.5) (layer "F.Cu") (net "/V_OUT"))
 (segment (start 157.725 114.75) (end 157.75 114.725) (width 0.5) (layer "F.Cu") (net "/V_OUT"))
 (segment (start 161.52 110.23) (end 162 110.23) (width 0.5) (layer "F.Cu") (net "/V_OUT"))
 (segment (start 160.25 111.5) (end 161.52 110.23) (width 0.5) (layer "F.Cu") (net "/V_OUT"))
 (segment (start 157.75 114) (end 157 113.25) (width 0.5) (layer "F.Cu") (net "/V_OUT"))
 (segment (start 157 112.25) (end 157.75 111.5) (width 0.5) (layer "F.Cu") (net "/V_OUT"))
 (segment (start 162.675 118.825) (end 163.625 117.875) (width 0.25) (layer "F.Cu") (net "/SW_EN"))
 (segment (start 160 108.5) (end 158.975 109.525) (width 0.25) (layer "F.Cu") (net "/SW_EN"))
 (segment (start 163.625 109.25) (end 162.875 108.5) (width 0.25) (layer "F.Cu") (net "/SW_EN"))
 (segment (start 161.2 118.825) (end 158.725 118.825) (width 0.25) (layer "F.Cu") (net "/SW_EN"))
 (segment (start 161.2 118.825) (end 162.675 118.825) (width 0.25) (layer "F.Cu") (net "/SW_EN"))
 (segment (start 158.975 109.525) (end 158.975 110.425) (width 0.25) (layer "F.Cu") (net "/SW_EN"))
 (segment (start 163.625 117.875) (end 163.625 109.25) (width 0.25) (layer "F.Cu") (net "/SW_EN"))
 (segment (start 158.725 118.825) (end 158.7 118.8) (width 0.25) (layer "F.Cu") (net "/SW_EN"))
 (segment (start 162.875 108.5) (end 160 108.5) (width 0.25) (layer "F.Cu") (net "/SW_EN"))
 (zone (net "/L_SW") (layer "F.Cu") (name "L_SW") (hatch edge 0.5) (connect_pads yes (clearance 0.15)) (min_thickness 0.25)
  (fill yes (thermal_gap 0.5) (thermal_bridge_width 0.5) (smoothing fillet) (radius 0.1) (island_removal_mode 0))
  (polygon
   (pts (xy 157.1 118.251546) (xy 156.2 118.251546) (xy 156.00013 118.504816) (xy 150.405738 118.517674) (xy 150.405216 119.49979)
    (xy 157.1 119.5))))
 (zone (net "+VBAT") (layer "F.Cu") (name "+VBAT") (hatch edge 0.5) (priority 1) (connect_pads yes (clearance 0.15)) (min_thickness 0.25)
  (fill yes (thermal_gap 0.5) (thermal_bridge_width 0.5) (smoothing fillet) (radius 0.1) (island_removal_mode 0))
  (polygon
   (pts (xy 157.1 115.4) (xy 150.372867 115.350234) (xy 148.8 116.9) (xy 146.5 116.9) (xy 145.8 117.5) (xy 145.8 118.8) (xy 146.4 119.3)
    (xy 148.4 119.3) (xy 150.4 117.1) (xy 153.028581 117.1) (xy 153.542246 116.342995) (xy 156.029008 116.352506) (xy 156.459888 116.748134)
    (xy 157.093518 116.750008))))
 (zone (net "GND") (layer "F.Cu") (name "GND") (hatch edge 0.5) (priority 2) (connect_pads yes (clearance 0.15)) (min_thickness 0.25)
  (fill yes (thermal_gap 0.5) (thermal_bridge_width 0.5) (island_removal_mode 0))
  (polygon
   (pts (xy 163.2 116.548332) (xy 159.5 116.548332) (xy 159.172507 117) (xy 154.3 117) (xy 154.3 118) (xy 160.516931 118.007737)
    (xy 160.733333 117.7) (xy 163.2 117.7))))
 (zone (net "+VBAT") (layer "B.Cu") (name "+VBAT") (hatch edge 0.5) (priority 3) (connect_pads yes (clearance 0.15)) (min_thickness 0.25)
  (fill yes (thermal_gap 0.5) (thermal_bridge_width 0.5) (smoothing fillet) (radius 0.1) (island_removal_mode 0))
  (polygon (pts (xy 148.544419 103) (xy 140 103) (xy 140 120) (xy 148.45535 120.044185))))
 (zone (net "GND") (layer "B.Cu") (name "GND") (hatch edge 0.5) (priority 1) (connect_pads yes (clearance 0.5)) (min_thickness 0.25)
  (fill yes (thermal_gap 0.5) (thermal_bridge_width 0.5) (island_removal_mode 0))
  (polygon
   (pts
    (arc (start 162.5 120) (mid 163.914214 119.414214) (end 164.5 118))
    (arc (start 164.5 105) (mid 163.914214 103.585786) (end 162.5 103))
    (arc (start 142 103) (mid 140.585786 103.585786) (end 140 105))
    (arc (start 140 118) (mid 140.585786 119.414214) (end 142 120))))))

